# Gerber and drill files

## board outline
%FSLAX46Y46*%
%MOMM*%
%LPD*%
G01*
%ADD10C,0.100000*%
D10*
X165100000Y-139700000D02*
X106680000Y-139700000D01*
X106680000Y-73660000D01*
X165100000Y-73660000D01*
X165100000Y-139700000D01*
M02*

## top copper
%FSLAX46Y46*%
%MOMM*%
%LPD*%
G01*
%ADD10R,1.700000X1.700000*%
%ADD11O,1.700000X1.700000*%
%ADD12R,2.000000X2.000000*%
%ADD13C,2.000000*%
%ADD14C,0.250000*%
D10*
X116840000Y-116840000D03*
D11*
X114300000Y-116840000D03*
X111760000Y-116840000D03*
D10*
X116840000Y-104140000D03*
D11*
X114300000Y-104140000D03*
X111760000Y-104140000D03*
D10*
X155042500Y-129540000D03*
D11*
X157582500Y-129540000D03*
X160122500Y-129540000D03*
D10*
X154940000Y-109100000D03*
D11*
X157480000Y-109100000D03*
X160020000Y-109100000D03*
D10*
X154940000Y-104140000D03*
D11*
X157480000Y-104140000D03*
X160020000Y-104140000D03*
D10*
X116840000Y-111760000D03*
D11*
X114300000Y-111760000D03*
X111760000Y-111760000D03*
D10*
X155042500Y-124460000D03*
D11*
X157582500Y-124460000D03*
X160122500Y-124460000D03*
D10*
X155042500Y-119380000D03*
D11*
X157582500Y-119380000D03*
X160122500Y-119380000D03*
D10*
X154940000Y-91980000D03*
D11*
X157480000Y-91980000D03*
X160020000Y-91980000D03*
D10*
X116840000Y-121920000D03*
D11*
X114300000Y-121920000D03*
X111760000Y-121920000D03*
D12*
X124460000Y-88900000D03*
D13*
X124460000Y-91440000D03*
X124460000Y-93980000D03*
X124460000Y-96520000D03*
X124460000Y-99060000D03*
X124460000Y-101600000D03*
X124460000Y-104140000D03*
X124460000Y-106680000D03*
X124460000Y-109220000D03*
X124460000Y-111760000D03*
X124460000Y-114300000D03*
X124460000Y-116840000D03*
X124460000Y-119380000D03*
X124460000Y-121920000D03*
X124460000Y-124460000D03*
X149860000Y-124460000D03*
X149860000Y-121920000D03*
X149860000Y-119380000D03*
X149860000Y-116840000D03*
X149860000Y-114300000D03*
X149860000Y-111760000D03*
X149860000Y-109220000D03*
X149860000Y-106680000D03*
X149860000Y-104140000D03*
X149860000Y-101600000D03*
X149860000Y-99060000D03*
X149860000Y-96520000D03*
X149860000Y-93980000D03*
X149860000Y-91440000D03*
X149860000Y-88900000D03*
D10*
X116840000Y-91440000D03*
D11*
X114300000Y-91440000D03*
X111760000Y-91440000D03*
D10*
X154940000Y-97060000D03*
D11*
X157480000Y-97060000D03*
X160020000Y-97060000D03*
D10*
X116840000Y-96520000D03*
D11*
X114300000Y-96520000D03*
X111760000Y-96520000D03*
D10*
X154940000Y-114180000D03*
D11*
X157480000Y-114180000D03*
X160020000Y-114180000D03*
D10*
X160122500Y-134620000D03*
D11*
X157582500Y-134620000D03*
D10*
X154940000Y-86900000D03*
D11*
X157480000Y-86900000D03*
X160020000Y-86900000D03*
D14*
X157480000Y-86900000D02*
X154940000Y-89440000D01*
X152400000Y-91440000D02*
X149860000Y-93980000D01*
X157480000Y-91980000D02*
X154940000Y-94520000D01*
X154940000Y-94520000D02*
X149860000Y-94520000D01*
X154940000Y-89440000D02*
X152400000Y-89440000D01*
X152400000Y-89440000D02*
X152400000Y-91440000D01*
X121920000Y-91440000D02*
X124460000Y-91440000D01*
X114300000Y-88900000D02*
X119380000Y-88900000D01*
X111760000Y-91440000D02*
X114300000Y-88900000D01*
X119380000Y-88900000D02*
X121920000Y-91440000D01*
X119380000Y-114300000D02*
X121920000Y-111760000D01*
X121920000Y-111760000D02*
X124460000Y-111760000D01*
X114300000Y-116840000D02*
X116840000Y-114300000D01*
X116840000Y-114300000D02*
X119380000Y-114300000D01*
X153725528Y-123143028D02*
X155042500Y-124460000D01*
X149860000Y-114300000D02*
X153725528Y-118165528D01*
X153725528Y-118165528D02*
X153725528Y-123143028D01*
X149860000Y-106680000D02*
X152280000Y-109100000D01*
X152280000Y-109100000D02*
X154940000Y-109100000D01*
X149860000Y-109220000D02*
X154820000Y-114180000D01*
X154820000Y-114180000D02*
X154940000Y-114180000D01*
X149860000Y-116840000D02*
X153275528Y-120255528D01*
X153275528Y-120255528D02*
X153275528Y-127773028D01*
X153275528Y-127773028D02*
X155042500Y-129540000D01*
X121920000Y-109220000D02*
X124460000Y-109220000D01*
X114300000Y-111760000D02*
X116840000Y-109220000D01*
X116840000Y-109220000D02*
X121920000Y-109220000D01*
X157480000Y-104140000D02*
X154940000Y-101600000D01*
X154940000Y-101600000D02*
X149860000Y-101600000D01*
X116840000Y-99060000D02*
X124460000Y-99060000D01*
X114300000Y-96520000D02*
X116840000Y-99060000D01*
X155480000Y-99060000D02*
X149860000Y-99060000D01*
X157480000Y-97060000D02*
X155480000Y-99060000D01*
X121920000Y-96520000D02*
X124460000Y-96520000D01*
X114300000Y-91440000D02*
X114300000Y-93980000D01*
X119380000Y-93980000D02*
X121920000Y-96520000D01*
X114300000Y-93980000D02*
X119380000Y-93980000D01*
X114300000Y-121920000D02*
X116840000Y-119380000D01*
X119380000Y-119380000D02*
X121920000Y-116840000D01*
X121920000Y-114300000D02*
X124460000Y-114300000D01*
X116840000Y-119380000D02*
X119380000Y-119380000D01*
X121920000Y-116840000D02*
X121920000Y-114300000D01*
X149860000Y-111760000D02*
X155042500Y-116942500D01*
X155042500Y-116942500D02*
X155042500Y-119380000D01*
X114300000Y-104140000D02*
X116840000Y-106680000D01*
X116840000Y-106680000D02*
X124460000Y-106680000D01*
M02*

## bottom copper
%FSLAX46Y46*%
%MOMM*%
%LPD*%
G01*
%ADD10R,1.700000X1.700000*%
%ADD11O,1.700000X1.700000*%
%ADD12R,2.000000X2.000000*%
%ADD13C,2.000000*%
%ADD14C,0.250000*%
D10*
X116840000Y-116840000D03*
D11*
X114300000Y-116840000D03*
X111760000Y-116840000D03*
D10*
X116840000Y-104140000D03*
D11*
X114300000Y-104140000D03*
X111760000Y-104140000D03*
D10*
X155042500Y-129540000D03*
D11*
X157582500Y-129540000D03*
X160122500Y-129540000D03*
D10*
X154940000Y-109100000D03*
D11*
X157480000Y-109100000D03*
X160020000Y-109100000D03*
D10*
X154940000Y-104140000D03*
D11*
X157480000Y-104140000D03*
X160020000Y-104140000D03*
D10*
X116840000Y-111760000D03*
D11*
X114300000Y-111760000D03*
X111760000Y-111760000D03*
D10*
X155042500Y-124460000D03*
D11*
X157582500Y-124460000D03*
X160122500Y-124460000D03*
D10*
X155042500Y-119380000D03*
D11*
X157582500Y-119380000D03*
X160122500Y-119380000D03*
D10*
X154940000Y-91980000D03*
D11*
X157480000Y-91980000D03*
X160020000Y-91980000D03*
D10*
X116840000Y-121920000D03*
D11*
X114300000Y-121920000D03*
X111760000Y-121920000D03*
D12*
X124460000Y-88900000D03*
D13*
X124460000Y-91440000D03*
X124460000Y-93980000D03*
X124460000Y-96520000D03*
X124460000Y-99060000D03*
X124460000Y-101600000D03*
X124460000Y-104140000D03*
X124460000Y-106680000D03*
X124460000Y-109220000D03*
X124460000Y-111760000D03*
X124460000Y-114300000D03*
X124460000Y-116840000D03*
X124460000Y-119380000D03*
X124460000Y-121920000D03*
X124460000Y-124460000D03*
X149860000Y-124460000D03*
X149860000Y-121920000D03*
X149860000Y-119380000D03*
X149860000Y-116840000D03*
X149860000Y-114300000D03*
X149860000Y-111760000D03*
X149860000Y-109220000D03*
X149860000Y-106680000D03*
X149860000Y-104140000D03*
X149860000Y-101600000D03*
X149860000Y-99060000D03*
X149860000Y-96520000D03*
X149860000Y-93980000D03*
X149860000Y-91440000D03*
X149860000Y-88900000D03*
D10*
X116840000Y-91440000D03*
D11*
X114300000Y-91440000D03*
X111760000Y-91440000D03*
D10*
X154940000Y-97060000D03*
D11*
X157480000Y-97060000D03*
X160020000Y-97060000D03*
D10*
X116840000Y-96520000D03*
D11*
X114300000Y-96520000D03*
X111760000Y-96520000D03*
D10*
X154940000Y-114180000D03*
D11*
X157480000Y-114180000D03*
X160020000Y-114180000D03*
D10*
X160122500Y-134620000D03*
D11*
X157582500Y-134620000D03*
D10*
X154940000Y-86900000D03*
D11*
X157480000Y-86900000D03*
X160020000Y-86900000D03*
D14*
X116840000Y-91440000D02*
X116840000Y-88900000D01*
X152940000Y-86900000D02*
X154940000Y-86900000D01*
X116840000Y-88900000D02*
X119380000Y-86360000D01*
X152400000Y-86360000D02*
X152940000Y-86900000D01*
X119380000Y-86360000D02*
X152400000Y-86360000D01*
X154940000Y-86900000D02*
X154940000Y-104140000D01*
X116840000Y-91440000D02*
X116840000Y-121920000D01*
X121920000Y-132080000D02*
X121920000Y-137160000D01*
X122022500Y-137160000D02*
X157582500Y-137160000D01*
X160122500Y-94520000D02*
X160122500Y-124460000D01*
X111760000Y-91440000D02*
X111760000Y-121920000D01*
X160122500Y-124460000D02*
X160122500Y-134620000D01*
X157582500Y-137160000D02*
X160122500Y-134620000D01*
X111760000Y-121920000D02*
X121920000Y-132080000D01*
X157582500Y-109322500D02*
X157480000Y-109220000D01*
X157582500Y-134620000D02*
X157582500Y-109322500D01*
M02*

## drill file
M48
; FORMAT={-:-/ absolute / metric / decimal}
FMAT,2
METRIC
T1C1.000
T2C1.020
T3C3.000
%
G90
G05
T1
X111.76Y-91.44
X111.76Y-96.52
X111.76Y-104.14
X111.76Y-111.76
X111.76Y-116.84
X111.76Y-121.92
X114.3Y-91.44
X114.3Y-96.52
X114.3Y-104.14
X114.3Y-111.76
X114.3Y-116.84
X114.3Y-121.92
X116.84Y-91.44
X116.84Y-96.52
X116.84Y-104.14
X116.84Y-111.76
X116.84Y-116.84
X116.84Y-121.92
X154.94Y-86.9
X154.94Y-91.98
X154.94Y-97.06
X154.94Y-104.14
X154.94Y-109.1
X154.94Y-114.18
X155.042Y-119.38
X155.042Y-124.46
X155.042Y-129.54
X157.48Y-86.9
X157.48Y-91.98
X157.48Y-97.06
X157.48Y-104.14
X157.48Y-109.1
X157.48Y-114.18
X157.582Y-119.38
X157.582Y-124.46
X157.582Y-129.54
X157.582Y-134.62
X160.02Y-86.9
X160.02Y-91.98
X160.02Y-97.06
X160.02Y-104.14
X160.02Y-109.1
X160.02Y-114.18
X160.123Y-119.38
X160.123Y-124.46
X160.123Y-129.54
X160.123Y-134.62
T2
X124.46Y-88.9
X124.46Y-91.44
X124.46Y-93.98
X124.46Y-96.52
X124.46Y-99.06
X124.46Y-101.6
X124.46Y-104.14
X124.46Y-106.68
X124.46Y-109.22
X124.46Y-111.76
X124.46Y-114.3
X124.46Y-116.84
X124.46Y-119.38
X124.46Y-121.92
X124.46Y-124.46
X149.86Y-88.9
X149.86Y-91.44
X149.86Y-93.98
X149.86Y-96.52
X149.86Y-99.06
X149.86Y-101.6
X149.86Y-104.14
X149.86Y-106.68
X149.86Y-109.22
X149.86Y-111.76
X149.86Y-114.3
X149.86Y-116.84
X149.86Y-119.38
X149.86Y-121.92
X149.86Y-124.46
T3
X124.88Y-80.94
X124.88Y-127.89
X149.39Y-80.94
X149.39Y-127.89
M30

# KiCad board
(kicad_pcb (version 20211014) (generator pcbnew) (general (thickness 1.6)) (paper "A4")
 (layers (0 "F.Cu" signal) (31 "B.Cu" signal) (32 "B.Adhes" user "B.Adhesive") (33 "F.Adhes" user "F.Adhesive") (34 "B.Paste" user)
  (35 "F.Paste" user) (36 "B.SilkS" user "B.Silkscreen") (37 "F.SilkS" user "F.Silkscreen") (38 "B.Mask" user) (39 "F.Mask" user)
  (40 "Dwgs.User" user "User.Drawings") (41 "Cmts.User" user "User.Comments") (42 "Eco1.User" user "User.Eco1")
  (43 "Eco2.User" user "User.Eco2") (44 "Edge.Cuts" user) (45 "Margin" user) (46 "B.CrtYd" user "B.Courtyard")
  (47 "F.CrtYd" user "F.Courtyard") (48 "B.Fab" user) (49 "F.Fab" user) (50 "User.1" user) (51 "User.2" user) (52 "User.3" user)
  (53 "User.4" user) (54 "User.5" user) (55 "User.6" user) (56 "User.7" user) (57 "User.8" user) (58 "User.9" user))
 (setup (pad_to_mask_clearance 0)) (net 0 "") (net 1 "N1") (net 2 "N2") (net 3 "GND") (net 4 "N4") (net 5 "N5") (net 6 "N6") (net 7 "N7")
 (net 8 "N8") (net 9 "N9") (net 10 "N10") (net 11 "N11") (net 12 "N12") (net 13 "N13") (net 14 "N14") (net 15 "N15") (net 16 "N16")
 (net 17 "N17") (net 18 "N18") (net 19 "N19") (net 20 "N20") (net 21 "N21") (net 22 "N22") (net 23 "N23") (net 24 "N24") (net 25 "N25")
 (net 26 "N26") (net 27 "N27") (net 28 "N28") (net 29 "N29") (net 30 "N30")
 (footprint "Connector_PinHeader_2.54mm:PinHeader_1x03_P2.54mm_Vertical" (layer "F.Cu") (at 116.84 116.84 -90)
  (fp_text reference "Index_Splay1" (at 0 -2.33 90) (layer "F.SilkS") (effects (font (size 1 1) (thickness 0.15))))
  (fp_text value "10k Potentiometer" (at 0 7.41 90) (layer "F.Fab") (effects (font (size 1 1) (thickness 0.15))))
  (pad "1" thru_hole rect (at 0 0 270) (size 1.7 1.7) (drill 1) (layers *.Cu *.Mask) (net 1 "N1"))
  (pad "2" thru_hole oval (at 0 2.54 270) (size 1.7 1.7) (drill 1) (layers *.Cu *.Mask) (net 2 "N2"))
  (pad "3" thru_hole oval (at 0 5.08 270) (size 1.7 1.7) (drill 1) (layers *.Cu *.Mask) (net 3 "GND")))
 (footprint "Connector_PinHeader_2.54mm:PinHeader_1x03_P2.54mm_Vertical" (layer "F.Cu") (at 116.84 104.14 -90)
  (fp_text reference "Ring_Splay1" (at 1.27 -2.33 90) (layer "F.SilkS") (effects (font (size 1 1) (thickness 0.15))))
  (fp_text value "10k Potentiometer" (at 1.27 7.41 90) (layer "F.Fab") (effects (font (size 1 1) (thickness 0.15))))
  (pad "1" thru_hole rect (at 0 0 270) (size 1.7 1.7) (drill 1) (layers *.Cu *.Mask) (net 1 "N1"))
  (pad "2" thru_hole oval (at 0 2.54 270) (size 1.7 1.7) (drill 1) (layers *.Cu *.Mask) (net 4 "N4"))
  (pad "3" thru_hole oval (at 0 5.08 270) (size 1.7 1.7) (drill 1) (layers *.Cu *.Mask) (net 3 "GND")))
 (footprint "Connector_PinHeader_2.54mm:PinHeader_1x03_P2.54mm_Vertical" (layer "F.Cu") (at 155.0425 129.54 90)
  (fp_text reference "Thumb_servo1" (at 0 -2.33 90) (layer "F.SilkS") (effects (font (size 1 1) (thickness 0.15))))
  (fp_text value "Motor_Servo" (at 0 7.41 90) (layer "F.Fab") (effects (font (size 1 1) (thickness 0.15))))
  (pad "1" thru_hole rect (at 0 0 90) (size 1.7 1.7) (drill 1) (layers *.Cu *.Mask) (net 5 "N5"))
  (pad "2" thru_hole oval (at 0 2.54 90) (size 1.7 1.7) (drill 1) (layers *.Cu *.Mask) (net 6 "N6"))
  (pad "3" thru_hole oval (at 0 5.08 90) (size 1.7 1.7) (drill 1) (layers *.Cu *.Mask) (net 3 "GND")))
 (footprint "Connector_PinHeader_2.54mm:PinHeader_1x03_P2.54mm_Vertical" (layer "F.Cu") (at 154.94 109.1 90)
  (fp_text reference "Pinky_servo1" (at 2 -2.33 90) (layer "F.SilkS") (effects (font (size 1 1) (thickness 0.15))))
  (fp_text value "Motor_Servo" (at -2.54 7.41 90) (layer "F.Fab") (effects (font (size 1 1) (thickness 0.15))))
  (pad "1" thru_hole rect (at 0 0 90) (size 1.7 1.7) (drill 1) (layers *.Cu *.Mask) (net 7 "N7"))
  (pad "2" thru_hole oval (at 0 2.54 90) (size 1.7 1.7) (drill 1) (layers *.Cu *.Mask) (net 6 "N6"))
  (pad "3" thru_hole oval (at 0 5.08 90) (size 1.7 1.7) (drill 1) (layers *.Cu *.Mask) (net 3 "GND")))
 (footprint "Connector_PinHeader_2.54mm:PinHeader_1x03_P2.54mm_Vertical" (layer "F.Cu") (at 154.94 104.14 90)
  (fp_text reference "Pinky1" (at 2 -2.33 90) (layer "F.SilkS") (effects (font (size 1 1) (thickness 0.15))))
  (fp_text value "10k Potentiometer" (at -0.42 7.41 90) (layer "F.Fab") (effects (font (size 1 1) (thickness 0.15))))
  (pad "1" thru_hole rect (at 0 0 90) (size 1.7 1.7) (drill 1) (layers *.Cu *.Mask) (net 1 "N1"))
  (pad "2" thru_hole oval (at 0 2.54 90) (size 1.7 1.7) (drill 1) (layers *.Cu *.Mask) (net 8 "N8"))
  (pad "3" thru_hole oval (at 0 5.08 90) (size 1.7 1.7) (drill 1) (layers *.Cu *.Mask) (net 3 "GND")))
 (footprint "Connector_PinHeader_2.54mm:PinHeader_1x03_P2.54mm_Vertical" (layer "F.Cu") (at 116.84 111.76 -90)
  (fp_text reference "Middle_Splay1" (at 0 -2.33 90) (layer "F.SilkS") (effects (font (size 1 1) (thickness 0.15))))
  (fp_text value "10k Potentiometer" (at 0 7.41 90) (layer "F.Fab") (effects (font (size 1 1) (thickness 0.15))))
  (pad "1" thru_hole rect (at 0 0 270) (size 1.7 1.7) (drill 1) (layers *.Cu *.Mask) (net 1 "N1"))
  (pad "2" thru_hole oval (at 0 2.54 270) (size 1.7 1.7) (drill 1) (layers *.Cu *.Mask) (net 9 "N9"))
  (pad "3" thru_hole oval (at 0 5.08 270) (size 1.7 1.7) (drill 1) (layers *.Cu *.Mask) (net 3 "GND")))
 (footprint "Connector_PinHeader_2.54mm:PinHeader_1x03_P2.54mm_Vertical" (layer "F.Cu") (at 155.0425 124.46 90)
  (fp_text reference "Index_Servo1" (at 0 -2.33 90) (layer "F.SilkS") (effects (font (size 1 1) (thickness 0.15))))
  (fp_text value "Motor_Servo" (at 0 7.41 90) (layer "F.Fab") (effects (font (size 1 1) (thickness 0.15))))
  (pad "1" thru_hole rect (at 0 0 90) (size 1.7 1.7) (drill 1) (layers *.Cu *.Mask) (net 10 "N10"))
  (pad "2" thru_hole oval (at 0 2.54 90) (size 1.7 1.7) (drill 1) (layers *.Cu *.Mask) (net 6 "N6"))
  (pad "3" thru_hole oval (at 0 5.08 90) (size 1.7 1.7) (drill 1) (layers *.Cu *.Mask) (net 3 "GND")))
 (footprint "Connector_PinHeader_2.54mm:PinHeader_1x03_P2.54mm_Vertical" (layer "F.Cu") (at 155.0425 119.38 90)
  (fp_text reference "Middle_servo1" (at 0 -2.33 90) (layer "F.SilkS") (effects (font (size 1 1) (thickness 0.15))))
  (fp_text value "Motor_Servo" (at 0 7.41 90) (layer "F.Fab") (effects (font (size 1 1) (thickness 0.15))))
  (pad "1" thru_hole rect (at 0 0 90) (size 1.7 1.7) (drill 1) (layers *.Cu *.Mask) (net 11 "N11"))
  (pad "2" thru_hole oval (at 0 2.54 90) (size 1.7 1.7) (drill 1) (layers *.Cu *.Mask) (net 6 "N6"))
  (pad "3" thru_hole oval (at 0 5.08 90) (size 1.7 1.7) (drill 1) (layers *.Cu *.Mask) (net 3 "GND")))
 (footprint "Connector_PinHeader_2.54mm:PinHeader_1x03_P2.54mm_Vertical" (layer "F.Cu") (at 154.94 91.98 90)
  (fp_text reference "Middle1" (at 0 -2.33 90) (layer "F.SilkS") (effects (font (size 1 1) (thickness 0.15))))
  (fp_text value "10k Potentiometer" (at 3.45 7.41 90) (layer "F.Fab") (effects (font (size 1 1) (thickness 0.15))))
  (pad "1" thru_hole rect (at 0 0 90) (size 1.7 1.7) (drill 1) (layers *.Cu *.Mask) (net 1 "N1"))
  (pad "2" thru_hole oval (at 0 2.54 90) (size 1.7 1.7) (drill 1) (layers *.Cu *.Mask) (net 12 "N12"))
  (pad "3" thru_hole oval (at 0 5.08 90) (size 1.7 1.7) (drill 1) (layers *.Cu *.Mask) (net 3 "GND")))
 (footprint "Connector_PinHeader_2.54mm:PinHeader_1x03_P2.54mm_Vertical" (layer "F.Cu") (at 116.84 121.92 -90)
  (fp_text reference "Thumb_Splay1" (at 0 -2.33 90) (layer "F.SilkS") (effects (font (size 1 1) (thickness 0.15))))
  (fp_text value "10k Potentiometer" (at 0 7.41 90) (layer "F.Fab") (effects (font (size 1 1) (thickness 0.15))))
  (pad "1" thru_hole rect (at 0 0 270) (size 1.7 1.7) (drill 1) (layers *.Cu *.Mask) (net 1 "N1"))
  (pad "2" thru_hole oval (at 0 2.54 270) (size 1.7 1.7) (drill 1) (layers *.Cu *.Mask) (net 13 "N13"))
  (pad "3" thru_hole oval (at 0 5.08 270) (size 1.7 1.7) (drill 1) (layers *.Cu *.Mask) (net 3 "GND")))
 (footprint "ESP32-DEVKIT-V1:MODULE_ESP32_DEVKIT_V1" (layer "F.Cu") (at 137.16 104.415)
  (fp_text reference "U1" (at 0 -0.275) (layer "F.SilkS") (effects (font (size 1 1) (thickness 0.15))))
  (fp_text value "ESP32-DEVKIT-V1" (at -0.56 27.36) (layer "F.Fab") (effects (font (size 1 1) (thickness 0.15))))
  (pad "" np_thru_hole circle (at -12.28 -23.475) (size 3 3) (drill 3) (layers *.Cu *.Mask))
  (pad "" np_thru_hole circle (at 12.23 23.475) (size 3 3) (drill 3) (layers *.Cu *.Mask))
  (pad "" np_thru_hole circle (at 12.23 -23.475) (size 3 3) (drill 3) (layers *.Cu *.Mask))
  (pad "" np_thru_hole circle (at -12.28 23.475) (size 3 3) (drill 3) (layers *.Cu *.Mask))
  (pad "1" thru_hole rect (at -12.7 -15.515) (size 2 2) (drill 1.02) (layers *.Cu *.Mask) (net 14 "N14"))
  (pad "2" thru_hole circle (at -12.7 -12.975) (size 2 2) (drill 1.02) (layers *.Cu *.Mask) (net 3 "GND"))
  (pad "3" thru_hole circle (at -12.7 -10.435) (size 2 2) (drill 1.02) (layers *.Cu *.Mask) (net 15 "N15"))
  (pad "4" thru_hole circle (at -12.7 -7.895) (size 2 2) (drill 1.02) (layers *.Cu *.Mask) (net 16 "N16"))
  (pad "5" thru_hole circle (at -12.7 -5.355) (size 2 2) (drill 1.02) (layers *.Cu *.Mask) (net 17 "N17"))
  (pad "6" thru_hole circle (at -12.7 -2.815) (size 2 2) (drill 1.02) (layers *.Cu *.Mask) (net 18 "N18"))
  (pad "7" thru_hole circle (at -12.7 -0.275) (size 2 2) (drill 1.02) (layers *.Cu *.Mask) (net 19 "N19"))
  (pad "8" thru_hole circle (at -12.7 2.265) (size 2 2) (drill 1.02) (layers *.Cu *.Mask) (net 4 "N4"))
  (pad "9" thru_hole circle (at -12.7 4.805) (size 2 2) (drill 1.02) (layers *.Cu *.Mask) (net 9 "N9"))
  (pad "10" thru_hole circle (at -12.7 7.345) (size 2 2) (drill 1.02) (layers *.Cu *.Mask) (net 2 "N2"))
  (pad "11" thru_hole circle (at -12.7 9.885) (size 2 2) (drill 1.02) (layers *.Cu *.Mask) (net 13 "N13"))
  (pad "12" thru_hole circle (at -12.7 12.425) (size 2 2) (drill 1.02) (layers *.Cu *.Mask) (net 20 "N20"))
  (pad "13" thru_hole circle (at -12.7 14.965) (size 2 2) (drill 1.02) (layers *.Cu *.Mask) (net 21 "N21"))
  (pad "14" thru_hole circle (at -12.7 17.505) (size 2 2) (drill 1.02) (layers *.Cu *.Mask) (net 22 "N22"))
  (pad "15" thru_hole circle (at -12.7 20.045) (size 2 2) (drill 1.02) (layers *.Cu *.Mask) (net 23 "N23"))
  (pad "16" thru_hole circle (at 12.7 20.045) (size 2 2) (drill 1.02) (layers *.Cu *.Mask) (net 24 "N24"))
  (pad "17" thru_hole circle (at 12.7 17.505) (size 2 2) (drill 1.02) (layers *.Cu *.Mask) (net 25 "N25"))
  (pad "18" thru_hole circle (at 12.7 14.965) (size 2 2) (drill 1.02) (layers *.Cu *.Mask) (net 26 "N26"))
  (pad "19" thru_hole circle (at 12.7 12.425) (size 2 2) (drill 1.02) (layers *.Cu *.Mask) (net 5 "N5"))
  (pad "20" thru_hole circle (at 12.7 9.885) (size 2 2) (drill 1.02) (layers *.Cu *.Mask) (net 10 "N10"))
  (pad "21" thru_hole circle (at 12.7 7.345) (size 2 2) (drill 1.02) (layers *.Cu *.Mask) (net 11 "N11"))
  (pad "22" thru_hole circle (at 12.7 4.805) (size 2 2) (drill 1.02) (layers *.Cu *.Mask) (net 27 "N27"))
  (pad "23" thru_hole circle (at 12.7 2.265) (size 2 2) (drill 1.02) (layers *.Cu *.Mask) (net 7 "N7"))
  (pad "24" thru_hole circle (at 12.7 -0.275) (size 2 2) (drill 1.02) (layers *.Cu *.Mask) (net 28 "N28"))
  (pad "25" thru_hole circle (at 12.7 -2.815) (size 2 2) (drill 1.02) (layers *.Cu *.Mask) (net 8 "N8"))
  (pad "26" thru_hole circle (at 12.7 -5.355) (size 2 2) (drill 1.02) (layers *.Cu *.Mask) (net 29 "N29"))
  (pad "27" thru_hole circle (at 12.7 -7.895) (size 2 2) (drill 1.02) (layers *.Cu *.Mask) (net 12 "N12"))
  (pad "28" thru_hole circle (at 12.7 -10.435) (size 2 2) (drill 1.02) (layers *.Cu *.Mask) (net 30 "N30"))
  (pad "29" thru_hole circle (at 12.7 -12.975) (size 2 2) (drill 1.02) (layers *.Cu *.Mask) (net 3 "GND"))
  (pad "30" thru_hole circle (at 12.7 -15.515) (size 2 2) (drill 1.02) (layers *.Cu *.Mask) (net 1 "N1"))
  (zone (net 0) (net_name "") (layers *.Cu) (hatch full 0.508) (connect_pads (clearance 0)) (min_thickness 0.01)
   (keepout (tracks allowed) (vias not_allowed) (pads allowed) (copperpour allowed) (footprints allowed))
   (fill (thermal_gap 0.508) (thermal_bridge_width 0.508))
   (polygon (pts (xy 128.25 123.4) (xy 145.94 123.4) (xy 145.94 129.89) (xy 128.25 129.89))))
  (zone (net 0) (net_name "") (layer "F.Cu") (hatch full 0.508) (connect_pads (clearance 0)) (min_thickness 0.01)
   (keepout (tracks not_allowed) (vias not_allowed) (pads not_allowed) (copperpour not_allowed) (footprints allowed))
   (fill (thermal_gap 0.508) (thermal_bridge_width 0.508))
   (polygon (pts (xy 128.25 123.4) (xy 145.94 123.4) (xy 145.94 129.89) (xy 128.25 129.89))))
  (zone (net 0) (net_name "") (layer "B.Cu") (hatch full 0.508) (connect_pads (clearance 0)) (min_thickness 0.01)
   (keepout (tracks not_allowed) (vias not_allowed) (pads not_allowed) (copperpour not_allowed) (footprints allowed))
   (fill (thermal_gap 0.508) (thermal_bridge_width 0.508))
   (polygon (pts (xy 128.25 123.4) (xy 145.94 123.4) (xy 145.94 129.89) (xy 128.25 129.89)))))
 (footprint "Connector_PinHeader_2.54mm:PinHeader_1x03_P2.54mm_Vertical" (layer "F.Cu") (at 116.84 91.44 -90)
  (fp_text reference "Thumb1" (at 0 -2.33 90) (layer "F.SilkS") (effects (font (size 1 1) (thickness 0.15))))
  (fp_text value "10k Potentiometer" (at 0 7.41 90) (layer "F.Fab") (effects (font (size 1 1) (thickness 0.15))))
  (pad "1" thru_hole rect (at 0 0 270) (size 1.7 1.7) (drill 1) (layers *.Cu *.Mask) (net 1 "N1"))
  (pad "2" thru_hole oval (at 0 2.54 270) (size 1.7 1.7) (drill 1) (layers *.Cu *.Mask) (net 16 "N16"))
  (pad "3" thru_hole oval (at 0 5.08 270) (size 1.7 1.7) (drill 1) (layers *.Cu *.Mask) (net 3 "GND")))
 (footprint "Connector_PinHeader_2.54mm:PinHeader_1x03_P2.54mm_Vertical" (layer "F.Cu") (at 154.94 97.06 90)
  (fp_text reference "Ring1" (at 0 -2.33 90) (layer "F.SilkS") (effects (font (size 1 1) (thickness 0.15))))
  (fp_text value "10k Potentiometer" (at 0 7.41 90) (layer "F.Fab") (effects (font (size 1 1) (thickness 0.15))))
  (pad "1" thru_hole rect (at 0 0 90) (size 1.7 1.7) (drill 1) (layers *.Cu *.Mask) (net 1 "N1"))
  (pad "2" thru_hole oval (at 0 2.54 90) (size 1.7 1.7) (drill 1) (layers *.Cu *.Mask) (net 29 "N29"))
  (pad "3" thru_hole oval (at 0 5.08 90) (size 1.7 1.7) (drill 1) (layers *.Cu *.Mask) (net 3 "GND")))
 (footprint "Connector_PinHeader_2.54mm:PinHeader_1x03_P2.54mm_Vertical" (layer "F.Cu") (at 116.84 96.52 -90)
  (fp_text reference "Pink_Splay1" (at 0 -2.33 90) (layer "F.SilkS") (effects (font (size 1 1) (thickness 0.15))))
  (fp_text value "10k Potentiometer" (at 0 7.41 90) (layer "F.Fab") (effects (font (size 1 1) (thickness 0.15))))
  (pad "1" thru_hole rect (at 0 0 270) (size 1.7 1.7) (drill 1) (layers *.Cu *.Mask) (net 1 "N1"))
  (pad "2" thru_hole oval (at 0 2.54 270) (size 1.7 1.7) (drill 1) (layers *.Cu *.Mask) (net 17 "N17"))
  (pad "3" thru_hole oval (at 0 5.08 270) (size 1.7 1.7) (drill 1) (layers *.Cu *.Mask) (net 3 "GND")))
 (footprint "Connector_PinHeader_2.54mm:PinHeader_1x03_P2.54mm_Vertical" (layer "F.Cu") (at 154.94 114.18 90)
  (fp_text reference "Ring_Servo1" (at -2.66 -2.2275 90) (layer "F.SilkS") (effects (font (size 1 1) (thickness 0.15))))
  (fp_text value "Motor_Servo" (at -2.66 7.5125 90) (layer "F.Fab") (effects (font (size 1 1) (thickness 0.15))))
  (pad "1" thru_hole rect (at 0 0 90) (size 1.7 1.7) (drill 1) (layers *.Cu *.Mask) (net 27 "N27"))
  (pad "2" thru_hole oval (at 0 2.54 90) (size 1.7 1.7) (drill 1) (layers *.Cu *.Mask) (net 6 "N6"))
  (pad "3" thru_hole oval (at 0 5.08 90) (size 1.7 1.7) (drill 1) (layers *.Cu *.Mask) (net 3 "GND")))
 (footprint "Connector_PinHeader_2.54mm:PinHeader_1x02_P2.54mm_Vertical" (layer "F.Cu") (at 160.1225 134.62 -90)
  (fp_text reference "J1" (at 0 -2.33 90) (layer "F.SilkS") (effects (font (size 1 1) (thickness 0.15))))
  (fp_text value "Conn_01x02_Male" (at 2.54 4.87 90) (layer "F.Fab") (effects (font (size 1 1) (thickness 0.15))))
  (pad "1" thru_hole rect (at 0 0 270) (size 1.7 1.7) (drill 1) (layers *.Cu *.Mask) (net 3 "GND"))
  (pad "2" thru_hole oval (at 0 2.54 270) (size 1.7 1.7) (drill 1) (layers *.Cu *.Mask) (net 6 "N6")))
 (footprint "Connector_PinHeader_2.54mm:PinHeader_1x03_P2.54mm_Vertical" (layer "F.Cu") (at 154.94 86.9 90)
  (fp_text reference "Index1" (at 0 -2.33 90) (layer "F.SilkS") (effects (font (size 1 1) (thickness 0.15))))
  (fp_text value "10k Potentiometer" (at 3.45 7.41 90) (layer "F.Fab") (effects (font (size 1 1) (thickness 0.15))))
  (pad "1" thru_hole rect (at 0 0 90) (size 1.7 1.7) (drill 1) (layers *.Cu *.Mask) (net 1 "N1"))
  (pad "2" thru_hole oval (at 0 2.54 90) (size 1.7 1.7) (drill 1) (layers *.Cu *.Mask) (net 30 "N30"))
  (pad "3" thru_hole oval (at 0 5.08 90) (size 1.7 1.7) (drill 1) (layers *.Cu *.Mask) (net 3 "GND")))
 (gr_poly (pts (xy 165.1 139.7) (xy 106.68 139.7) (xy 106.68 73.66) (xy 165.1 73.66)) (layer "Edge.Cuts") (width 0.1) (fill none))
 (segment (start 116.84 91.44) (end 116.84 88.9) (width 0.25) (layer "B.Cu") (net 1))
 (segment (start 152.94 86.9) (end 154.94 86.9) (width 0.25) (layer "B.Cu") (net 1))
 (segment (start 116.84 88.9) (end 119.38 86.36) (width 0.25) (layer "B.Cu") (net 1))
 (segment (start 152.4 86.36) (end 152.94 86.9) (width 0.25) (layer "B.Cu") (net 1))
 (segment (start 119.38 86.36) (end 152.4 86.36) (width 0.25) (layer "B.Cu") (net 1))
 (segment (start 154.94 86.9) (end 154.94 104.14) (width 0.25) (layer "B.Cu") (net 1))
 (segment (start 116.84 91.44) (end 116.84 121.92) (width 0.25) (layer "B.Cu") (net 1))
 (segment (start 157.48 86.9) (end 154.94 89.44) (width 0.25) (layer "F.Cu") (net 30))
 (segment (start 152.4 91.44) (end 149.86 93.98) (width 0.25) (layer "F.Cu") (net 30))
 (segment (start 157.48 91.98) (end 154.94 94.52) (width 0.25) (layer "F.Cu") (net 30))
 (segment (start 154.94 94.52) (end 149.86 94.52) (width 0.25) (layer "F.Cu") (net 30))
 (segment (start 154.94 89.44) (end 152.4 89.44) (width 0.25) (layer "F.Cu") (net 30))
 (segment (start 152.4 89.44) (end 152.4 91.44) (width 0.25) (layer "F.Cu") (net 30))
 (segment (start 121.92 91.44) (end 124.46 91.44) (width 0.25) (layer "F.Cu") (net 3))
 (segment (start 114.3 88.9) (end 119.38 88.9) (width 0.25) (layer "F.Cu") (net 3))
 (segment (start 111.76 91.44) (end 114.3 88.9) (width 0.25) (layer "F.Cu") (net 3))
 (segment (start 119.38 88.9) (end 121.92 91.44) (width 0.25) (layer "F.Cu") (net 3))
 (segment (start 121.92 132.08) (end 121.92 137.16) (width 0.25) (layer "B.Cu") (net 3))
 (segment (start 122.0225 137.16) (end 157.5825 137.16) (width 0.25) (layer "B.Cu") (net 3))
 (segment (start 160.1225 94.52) (end 160.1225 124.46) (width 0.25) (layer "B.Cu") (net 3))
 (segment (start 111.76 91.44) (end 111.76 121.92) (width 0.25) (layer "B.Cu") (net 3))
 (segment (start 160.1225 124.46) (end 160.1225 134.62) (width 0.25) (layer "B.Cu") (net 3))
 (segment (start 157.5825 137.16) (end 160.1225 134.62) (width 0.25) (layer "B.Cu") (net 3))
 (segment (start 111.76 121.92) (end 121.92 132.08) (width 0.25) (layer "B.Cu") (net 3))
 (segment (start 119.38 114.3) (end 121.92 111.76) (width 0.25) (layer "F.Cu") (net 2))
 (segment (start 121.92 111.76) (end 124.46 111.76) (width 0.25) (layer "F.Cu") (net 2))
 (segment (start 114.3 116.84) (end 116.84 114.3) (width 0.25) (layer "F.Cu") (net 2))
 (segment (start 116.84 114.3) (end 119.38 114.3) (width 0.25) (layer "F.Cu") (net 2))
 (segment (start 153.725528 123.143028) (end 155.0425 124.46) (width 0.25) (layer "F.Cu") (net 10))
 (segment (start 149.86 114.3) (end 153.725528 118.165528) (width 0.25) (layer "F.Cu") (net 10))
 (segment (start 153.725528 118.165528) (end 153.725528 123.143028) (width 0.25) (layer "F.Cu") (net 10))
 (segment (start 149.86 106.68) (end 152.28 109.1) (width 0.25) (layer "F.Cu") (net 7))
 (segment (start 152.28 109.1) (end 154.94 109.1) (width 0.25) (layer "F.Cu") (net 7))
 (segment (start 149.86 109.22) (end 154.82 114.18) (width 0.25) (layer "F.Cu") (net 27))
 (segment (start 154.82 114.18) (end 154.94 114.18) (width 0.25) (layer "F.Cu") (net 27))
 (segment (start 149.86 116.84) (end 153.275528 120.255528) (width 0.25) (layer "F.Cu") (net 5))
 (segment (start 153.275528 120.255528) (end 153.275528 127.773028) (width 0.25) (layer "F.Cu") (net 5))
 (segment (start 153.275528 127.773028) (end 155.0425 129.54) (width 0.25) (layer "F.Cu") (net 5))
 (segment (start 121.92 109.22) (end 124.46 109.22) (width 0.25) (layer "F.Cu") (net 9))
 (segment (start 114.3 111.76) (end 116.84 109.22) (width 0.25) (layer "F.Cu") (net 9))
 (segment (start 116.84 109.22) (end 121.92 109.22) (width 0.25) (layer "F.Cu") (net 9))
 (segment (start 157.48 104.14) (end 154.94 101.6) (width 0.25) (layer "F.Cu") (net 8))
 (segment (start 154.94 101.6) (end 149.86 101.6) (width 0.25) (layer "F.Cu") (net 8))
 (segment (start 116.84 99.06) (end 124.46 99.06) (width 0.25) (layer "F.Cu") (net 17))
 (segment (start 114.3 96.52) (end 116.84 99.06) (width 0.25) (layer "F.Cu") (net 17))
 (segment (start 155.48 99.06) (end 149.86 99.06) (width 0.25) (layer "F.Cu") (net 29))
 (segment (start 157.48 97.06) (end 155.48 99.06) (width 0.25) (layer "F.Cu") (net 29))
 (segment (start 121.92 96.52) (end 124.46 96.52) (width 0.25) (layer "F.Cu") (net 16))
 (segment (start 114.3 91.44) (end 114.3 93.98) (width 0.25) (layer "F.Cu") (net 16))
 (segment (start 119.38 93.98) (end 121.92 96.52) (width 0.25) (layer "F.Cu") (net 16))
 (segment (start 114.3 93.98) (end 119.38 93.98) (width 0.25) (layer "F.Cu") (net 16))
 (segment (start 114.3 121.92) (end 116.84 119.38) (width 0.25) (layer "F.Cu") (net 13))
 (segment (start 119.38 119.38) (end 121.92 116.84) (width 0.25) (layer "F.Cu") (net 13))
 (segment (start 121.92 114.3) (end 124.46 114.3) (width 0.25) (layer "F.Cu") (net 13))
 (segment (start 116.84 119.38) (end 119.38 119.38) (width 0.25) (layer "F.Cu") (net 13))
 (segment (start 121.92 116.84) (end 121.92 114.3) (width 0.25) (layer "F.Cu") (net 13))
 (segment (start 157.5825 109.3225) (end 157.48 109.22) (width 0.25) (layer "B.Cu") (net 6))
 (segment (start 157.5825 134.62) (end 157.5825 109.3225) (width 0.25) (layer "B.Cu") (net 6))
 (segment (start 149.86 111.76) (end 155.0425 116.9425) (width 0.25) (layer "F.Cu") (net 11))
 (segment (start 155.0425 116.9425) (end 155.0425 119.38) (width 0.25) (layer "F.Cu") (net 11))
 (segment (start 114.3 104.14) (end 116.84 106.68) (width 0.25) (layer "F.Cu") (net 4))
 (segment (start 116.84 106.68) (end 124.46 106.68) (width 0.25) (layer "F.Cu") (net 4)))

